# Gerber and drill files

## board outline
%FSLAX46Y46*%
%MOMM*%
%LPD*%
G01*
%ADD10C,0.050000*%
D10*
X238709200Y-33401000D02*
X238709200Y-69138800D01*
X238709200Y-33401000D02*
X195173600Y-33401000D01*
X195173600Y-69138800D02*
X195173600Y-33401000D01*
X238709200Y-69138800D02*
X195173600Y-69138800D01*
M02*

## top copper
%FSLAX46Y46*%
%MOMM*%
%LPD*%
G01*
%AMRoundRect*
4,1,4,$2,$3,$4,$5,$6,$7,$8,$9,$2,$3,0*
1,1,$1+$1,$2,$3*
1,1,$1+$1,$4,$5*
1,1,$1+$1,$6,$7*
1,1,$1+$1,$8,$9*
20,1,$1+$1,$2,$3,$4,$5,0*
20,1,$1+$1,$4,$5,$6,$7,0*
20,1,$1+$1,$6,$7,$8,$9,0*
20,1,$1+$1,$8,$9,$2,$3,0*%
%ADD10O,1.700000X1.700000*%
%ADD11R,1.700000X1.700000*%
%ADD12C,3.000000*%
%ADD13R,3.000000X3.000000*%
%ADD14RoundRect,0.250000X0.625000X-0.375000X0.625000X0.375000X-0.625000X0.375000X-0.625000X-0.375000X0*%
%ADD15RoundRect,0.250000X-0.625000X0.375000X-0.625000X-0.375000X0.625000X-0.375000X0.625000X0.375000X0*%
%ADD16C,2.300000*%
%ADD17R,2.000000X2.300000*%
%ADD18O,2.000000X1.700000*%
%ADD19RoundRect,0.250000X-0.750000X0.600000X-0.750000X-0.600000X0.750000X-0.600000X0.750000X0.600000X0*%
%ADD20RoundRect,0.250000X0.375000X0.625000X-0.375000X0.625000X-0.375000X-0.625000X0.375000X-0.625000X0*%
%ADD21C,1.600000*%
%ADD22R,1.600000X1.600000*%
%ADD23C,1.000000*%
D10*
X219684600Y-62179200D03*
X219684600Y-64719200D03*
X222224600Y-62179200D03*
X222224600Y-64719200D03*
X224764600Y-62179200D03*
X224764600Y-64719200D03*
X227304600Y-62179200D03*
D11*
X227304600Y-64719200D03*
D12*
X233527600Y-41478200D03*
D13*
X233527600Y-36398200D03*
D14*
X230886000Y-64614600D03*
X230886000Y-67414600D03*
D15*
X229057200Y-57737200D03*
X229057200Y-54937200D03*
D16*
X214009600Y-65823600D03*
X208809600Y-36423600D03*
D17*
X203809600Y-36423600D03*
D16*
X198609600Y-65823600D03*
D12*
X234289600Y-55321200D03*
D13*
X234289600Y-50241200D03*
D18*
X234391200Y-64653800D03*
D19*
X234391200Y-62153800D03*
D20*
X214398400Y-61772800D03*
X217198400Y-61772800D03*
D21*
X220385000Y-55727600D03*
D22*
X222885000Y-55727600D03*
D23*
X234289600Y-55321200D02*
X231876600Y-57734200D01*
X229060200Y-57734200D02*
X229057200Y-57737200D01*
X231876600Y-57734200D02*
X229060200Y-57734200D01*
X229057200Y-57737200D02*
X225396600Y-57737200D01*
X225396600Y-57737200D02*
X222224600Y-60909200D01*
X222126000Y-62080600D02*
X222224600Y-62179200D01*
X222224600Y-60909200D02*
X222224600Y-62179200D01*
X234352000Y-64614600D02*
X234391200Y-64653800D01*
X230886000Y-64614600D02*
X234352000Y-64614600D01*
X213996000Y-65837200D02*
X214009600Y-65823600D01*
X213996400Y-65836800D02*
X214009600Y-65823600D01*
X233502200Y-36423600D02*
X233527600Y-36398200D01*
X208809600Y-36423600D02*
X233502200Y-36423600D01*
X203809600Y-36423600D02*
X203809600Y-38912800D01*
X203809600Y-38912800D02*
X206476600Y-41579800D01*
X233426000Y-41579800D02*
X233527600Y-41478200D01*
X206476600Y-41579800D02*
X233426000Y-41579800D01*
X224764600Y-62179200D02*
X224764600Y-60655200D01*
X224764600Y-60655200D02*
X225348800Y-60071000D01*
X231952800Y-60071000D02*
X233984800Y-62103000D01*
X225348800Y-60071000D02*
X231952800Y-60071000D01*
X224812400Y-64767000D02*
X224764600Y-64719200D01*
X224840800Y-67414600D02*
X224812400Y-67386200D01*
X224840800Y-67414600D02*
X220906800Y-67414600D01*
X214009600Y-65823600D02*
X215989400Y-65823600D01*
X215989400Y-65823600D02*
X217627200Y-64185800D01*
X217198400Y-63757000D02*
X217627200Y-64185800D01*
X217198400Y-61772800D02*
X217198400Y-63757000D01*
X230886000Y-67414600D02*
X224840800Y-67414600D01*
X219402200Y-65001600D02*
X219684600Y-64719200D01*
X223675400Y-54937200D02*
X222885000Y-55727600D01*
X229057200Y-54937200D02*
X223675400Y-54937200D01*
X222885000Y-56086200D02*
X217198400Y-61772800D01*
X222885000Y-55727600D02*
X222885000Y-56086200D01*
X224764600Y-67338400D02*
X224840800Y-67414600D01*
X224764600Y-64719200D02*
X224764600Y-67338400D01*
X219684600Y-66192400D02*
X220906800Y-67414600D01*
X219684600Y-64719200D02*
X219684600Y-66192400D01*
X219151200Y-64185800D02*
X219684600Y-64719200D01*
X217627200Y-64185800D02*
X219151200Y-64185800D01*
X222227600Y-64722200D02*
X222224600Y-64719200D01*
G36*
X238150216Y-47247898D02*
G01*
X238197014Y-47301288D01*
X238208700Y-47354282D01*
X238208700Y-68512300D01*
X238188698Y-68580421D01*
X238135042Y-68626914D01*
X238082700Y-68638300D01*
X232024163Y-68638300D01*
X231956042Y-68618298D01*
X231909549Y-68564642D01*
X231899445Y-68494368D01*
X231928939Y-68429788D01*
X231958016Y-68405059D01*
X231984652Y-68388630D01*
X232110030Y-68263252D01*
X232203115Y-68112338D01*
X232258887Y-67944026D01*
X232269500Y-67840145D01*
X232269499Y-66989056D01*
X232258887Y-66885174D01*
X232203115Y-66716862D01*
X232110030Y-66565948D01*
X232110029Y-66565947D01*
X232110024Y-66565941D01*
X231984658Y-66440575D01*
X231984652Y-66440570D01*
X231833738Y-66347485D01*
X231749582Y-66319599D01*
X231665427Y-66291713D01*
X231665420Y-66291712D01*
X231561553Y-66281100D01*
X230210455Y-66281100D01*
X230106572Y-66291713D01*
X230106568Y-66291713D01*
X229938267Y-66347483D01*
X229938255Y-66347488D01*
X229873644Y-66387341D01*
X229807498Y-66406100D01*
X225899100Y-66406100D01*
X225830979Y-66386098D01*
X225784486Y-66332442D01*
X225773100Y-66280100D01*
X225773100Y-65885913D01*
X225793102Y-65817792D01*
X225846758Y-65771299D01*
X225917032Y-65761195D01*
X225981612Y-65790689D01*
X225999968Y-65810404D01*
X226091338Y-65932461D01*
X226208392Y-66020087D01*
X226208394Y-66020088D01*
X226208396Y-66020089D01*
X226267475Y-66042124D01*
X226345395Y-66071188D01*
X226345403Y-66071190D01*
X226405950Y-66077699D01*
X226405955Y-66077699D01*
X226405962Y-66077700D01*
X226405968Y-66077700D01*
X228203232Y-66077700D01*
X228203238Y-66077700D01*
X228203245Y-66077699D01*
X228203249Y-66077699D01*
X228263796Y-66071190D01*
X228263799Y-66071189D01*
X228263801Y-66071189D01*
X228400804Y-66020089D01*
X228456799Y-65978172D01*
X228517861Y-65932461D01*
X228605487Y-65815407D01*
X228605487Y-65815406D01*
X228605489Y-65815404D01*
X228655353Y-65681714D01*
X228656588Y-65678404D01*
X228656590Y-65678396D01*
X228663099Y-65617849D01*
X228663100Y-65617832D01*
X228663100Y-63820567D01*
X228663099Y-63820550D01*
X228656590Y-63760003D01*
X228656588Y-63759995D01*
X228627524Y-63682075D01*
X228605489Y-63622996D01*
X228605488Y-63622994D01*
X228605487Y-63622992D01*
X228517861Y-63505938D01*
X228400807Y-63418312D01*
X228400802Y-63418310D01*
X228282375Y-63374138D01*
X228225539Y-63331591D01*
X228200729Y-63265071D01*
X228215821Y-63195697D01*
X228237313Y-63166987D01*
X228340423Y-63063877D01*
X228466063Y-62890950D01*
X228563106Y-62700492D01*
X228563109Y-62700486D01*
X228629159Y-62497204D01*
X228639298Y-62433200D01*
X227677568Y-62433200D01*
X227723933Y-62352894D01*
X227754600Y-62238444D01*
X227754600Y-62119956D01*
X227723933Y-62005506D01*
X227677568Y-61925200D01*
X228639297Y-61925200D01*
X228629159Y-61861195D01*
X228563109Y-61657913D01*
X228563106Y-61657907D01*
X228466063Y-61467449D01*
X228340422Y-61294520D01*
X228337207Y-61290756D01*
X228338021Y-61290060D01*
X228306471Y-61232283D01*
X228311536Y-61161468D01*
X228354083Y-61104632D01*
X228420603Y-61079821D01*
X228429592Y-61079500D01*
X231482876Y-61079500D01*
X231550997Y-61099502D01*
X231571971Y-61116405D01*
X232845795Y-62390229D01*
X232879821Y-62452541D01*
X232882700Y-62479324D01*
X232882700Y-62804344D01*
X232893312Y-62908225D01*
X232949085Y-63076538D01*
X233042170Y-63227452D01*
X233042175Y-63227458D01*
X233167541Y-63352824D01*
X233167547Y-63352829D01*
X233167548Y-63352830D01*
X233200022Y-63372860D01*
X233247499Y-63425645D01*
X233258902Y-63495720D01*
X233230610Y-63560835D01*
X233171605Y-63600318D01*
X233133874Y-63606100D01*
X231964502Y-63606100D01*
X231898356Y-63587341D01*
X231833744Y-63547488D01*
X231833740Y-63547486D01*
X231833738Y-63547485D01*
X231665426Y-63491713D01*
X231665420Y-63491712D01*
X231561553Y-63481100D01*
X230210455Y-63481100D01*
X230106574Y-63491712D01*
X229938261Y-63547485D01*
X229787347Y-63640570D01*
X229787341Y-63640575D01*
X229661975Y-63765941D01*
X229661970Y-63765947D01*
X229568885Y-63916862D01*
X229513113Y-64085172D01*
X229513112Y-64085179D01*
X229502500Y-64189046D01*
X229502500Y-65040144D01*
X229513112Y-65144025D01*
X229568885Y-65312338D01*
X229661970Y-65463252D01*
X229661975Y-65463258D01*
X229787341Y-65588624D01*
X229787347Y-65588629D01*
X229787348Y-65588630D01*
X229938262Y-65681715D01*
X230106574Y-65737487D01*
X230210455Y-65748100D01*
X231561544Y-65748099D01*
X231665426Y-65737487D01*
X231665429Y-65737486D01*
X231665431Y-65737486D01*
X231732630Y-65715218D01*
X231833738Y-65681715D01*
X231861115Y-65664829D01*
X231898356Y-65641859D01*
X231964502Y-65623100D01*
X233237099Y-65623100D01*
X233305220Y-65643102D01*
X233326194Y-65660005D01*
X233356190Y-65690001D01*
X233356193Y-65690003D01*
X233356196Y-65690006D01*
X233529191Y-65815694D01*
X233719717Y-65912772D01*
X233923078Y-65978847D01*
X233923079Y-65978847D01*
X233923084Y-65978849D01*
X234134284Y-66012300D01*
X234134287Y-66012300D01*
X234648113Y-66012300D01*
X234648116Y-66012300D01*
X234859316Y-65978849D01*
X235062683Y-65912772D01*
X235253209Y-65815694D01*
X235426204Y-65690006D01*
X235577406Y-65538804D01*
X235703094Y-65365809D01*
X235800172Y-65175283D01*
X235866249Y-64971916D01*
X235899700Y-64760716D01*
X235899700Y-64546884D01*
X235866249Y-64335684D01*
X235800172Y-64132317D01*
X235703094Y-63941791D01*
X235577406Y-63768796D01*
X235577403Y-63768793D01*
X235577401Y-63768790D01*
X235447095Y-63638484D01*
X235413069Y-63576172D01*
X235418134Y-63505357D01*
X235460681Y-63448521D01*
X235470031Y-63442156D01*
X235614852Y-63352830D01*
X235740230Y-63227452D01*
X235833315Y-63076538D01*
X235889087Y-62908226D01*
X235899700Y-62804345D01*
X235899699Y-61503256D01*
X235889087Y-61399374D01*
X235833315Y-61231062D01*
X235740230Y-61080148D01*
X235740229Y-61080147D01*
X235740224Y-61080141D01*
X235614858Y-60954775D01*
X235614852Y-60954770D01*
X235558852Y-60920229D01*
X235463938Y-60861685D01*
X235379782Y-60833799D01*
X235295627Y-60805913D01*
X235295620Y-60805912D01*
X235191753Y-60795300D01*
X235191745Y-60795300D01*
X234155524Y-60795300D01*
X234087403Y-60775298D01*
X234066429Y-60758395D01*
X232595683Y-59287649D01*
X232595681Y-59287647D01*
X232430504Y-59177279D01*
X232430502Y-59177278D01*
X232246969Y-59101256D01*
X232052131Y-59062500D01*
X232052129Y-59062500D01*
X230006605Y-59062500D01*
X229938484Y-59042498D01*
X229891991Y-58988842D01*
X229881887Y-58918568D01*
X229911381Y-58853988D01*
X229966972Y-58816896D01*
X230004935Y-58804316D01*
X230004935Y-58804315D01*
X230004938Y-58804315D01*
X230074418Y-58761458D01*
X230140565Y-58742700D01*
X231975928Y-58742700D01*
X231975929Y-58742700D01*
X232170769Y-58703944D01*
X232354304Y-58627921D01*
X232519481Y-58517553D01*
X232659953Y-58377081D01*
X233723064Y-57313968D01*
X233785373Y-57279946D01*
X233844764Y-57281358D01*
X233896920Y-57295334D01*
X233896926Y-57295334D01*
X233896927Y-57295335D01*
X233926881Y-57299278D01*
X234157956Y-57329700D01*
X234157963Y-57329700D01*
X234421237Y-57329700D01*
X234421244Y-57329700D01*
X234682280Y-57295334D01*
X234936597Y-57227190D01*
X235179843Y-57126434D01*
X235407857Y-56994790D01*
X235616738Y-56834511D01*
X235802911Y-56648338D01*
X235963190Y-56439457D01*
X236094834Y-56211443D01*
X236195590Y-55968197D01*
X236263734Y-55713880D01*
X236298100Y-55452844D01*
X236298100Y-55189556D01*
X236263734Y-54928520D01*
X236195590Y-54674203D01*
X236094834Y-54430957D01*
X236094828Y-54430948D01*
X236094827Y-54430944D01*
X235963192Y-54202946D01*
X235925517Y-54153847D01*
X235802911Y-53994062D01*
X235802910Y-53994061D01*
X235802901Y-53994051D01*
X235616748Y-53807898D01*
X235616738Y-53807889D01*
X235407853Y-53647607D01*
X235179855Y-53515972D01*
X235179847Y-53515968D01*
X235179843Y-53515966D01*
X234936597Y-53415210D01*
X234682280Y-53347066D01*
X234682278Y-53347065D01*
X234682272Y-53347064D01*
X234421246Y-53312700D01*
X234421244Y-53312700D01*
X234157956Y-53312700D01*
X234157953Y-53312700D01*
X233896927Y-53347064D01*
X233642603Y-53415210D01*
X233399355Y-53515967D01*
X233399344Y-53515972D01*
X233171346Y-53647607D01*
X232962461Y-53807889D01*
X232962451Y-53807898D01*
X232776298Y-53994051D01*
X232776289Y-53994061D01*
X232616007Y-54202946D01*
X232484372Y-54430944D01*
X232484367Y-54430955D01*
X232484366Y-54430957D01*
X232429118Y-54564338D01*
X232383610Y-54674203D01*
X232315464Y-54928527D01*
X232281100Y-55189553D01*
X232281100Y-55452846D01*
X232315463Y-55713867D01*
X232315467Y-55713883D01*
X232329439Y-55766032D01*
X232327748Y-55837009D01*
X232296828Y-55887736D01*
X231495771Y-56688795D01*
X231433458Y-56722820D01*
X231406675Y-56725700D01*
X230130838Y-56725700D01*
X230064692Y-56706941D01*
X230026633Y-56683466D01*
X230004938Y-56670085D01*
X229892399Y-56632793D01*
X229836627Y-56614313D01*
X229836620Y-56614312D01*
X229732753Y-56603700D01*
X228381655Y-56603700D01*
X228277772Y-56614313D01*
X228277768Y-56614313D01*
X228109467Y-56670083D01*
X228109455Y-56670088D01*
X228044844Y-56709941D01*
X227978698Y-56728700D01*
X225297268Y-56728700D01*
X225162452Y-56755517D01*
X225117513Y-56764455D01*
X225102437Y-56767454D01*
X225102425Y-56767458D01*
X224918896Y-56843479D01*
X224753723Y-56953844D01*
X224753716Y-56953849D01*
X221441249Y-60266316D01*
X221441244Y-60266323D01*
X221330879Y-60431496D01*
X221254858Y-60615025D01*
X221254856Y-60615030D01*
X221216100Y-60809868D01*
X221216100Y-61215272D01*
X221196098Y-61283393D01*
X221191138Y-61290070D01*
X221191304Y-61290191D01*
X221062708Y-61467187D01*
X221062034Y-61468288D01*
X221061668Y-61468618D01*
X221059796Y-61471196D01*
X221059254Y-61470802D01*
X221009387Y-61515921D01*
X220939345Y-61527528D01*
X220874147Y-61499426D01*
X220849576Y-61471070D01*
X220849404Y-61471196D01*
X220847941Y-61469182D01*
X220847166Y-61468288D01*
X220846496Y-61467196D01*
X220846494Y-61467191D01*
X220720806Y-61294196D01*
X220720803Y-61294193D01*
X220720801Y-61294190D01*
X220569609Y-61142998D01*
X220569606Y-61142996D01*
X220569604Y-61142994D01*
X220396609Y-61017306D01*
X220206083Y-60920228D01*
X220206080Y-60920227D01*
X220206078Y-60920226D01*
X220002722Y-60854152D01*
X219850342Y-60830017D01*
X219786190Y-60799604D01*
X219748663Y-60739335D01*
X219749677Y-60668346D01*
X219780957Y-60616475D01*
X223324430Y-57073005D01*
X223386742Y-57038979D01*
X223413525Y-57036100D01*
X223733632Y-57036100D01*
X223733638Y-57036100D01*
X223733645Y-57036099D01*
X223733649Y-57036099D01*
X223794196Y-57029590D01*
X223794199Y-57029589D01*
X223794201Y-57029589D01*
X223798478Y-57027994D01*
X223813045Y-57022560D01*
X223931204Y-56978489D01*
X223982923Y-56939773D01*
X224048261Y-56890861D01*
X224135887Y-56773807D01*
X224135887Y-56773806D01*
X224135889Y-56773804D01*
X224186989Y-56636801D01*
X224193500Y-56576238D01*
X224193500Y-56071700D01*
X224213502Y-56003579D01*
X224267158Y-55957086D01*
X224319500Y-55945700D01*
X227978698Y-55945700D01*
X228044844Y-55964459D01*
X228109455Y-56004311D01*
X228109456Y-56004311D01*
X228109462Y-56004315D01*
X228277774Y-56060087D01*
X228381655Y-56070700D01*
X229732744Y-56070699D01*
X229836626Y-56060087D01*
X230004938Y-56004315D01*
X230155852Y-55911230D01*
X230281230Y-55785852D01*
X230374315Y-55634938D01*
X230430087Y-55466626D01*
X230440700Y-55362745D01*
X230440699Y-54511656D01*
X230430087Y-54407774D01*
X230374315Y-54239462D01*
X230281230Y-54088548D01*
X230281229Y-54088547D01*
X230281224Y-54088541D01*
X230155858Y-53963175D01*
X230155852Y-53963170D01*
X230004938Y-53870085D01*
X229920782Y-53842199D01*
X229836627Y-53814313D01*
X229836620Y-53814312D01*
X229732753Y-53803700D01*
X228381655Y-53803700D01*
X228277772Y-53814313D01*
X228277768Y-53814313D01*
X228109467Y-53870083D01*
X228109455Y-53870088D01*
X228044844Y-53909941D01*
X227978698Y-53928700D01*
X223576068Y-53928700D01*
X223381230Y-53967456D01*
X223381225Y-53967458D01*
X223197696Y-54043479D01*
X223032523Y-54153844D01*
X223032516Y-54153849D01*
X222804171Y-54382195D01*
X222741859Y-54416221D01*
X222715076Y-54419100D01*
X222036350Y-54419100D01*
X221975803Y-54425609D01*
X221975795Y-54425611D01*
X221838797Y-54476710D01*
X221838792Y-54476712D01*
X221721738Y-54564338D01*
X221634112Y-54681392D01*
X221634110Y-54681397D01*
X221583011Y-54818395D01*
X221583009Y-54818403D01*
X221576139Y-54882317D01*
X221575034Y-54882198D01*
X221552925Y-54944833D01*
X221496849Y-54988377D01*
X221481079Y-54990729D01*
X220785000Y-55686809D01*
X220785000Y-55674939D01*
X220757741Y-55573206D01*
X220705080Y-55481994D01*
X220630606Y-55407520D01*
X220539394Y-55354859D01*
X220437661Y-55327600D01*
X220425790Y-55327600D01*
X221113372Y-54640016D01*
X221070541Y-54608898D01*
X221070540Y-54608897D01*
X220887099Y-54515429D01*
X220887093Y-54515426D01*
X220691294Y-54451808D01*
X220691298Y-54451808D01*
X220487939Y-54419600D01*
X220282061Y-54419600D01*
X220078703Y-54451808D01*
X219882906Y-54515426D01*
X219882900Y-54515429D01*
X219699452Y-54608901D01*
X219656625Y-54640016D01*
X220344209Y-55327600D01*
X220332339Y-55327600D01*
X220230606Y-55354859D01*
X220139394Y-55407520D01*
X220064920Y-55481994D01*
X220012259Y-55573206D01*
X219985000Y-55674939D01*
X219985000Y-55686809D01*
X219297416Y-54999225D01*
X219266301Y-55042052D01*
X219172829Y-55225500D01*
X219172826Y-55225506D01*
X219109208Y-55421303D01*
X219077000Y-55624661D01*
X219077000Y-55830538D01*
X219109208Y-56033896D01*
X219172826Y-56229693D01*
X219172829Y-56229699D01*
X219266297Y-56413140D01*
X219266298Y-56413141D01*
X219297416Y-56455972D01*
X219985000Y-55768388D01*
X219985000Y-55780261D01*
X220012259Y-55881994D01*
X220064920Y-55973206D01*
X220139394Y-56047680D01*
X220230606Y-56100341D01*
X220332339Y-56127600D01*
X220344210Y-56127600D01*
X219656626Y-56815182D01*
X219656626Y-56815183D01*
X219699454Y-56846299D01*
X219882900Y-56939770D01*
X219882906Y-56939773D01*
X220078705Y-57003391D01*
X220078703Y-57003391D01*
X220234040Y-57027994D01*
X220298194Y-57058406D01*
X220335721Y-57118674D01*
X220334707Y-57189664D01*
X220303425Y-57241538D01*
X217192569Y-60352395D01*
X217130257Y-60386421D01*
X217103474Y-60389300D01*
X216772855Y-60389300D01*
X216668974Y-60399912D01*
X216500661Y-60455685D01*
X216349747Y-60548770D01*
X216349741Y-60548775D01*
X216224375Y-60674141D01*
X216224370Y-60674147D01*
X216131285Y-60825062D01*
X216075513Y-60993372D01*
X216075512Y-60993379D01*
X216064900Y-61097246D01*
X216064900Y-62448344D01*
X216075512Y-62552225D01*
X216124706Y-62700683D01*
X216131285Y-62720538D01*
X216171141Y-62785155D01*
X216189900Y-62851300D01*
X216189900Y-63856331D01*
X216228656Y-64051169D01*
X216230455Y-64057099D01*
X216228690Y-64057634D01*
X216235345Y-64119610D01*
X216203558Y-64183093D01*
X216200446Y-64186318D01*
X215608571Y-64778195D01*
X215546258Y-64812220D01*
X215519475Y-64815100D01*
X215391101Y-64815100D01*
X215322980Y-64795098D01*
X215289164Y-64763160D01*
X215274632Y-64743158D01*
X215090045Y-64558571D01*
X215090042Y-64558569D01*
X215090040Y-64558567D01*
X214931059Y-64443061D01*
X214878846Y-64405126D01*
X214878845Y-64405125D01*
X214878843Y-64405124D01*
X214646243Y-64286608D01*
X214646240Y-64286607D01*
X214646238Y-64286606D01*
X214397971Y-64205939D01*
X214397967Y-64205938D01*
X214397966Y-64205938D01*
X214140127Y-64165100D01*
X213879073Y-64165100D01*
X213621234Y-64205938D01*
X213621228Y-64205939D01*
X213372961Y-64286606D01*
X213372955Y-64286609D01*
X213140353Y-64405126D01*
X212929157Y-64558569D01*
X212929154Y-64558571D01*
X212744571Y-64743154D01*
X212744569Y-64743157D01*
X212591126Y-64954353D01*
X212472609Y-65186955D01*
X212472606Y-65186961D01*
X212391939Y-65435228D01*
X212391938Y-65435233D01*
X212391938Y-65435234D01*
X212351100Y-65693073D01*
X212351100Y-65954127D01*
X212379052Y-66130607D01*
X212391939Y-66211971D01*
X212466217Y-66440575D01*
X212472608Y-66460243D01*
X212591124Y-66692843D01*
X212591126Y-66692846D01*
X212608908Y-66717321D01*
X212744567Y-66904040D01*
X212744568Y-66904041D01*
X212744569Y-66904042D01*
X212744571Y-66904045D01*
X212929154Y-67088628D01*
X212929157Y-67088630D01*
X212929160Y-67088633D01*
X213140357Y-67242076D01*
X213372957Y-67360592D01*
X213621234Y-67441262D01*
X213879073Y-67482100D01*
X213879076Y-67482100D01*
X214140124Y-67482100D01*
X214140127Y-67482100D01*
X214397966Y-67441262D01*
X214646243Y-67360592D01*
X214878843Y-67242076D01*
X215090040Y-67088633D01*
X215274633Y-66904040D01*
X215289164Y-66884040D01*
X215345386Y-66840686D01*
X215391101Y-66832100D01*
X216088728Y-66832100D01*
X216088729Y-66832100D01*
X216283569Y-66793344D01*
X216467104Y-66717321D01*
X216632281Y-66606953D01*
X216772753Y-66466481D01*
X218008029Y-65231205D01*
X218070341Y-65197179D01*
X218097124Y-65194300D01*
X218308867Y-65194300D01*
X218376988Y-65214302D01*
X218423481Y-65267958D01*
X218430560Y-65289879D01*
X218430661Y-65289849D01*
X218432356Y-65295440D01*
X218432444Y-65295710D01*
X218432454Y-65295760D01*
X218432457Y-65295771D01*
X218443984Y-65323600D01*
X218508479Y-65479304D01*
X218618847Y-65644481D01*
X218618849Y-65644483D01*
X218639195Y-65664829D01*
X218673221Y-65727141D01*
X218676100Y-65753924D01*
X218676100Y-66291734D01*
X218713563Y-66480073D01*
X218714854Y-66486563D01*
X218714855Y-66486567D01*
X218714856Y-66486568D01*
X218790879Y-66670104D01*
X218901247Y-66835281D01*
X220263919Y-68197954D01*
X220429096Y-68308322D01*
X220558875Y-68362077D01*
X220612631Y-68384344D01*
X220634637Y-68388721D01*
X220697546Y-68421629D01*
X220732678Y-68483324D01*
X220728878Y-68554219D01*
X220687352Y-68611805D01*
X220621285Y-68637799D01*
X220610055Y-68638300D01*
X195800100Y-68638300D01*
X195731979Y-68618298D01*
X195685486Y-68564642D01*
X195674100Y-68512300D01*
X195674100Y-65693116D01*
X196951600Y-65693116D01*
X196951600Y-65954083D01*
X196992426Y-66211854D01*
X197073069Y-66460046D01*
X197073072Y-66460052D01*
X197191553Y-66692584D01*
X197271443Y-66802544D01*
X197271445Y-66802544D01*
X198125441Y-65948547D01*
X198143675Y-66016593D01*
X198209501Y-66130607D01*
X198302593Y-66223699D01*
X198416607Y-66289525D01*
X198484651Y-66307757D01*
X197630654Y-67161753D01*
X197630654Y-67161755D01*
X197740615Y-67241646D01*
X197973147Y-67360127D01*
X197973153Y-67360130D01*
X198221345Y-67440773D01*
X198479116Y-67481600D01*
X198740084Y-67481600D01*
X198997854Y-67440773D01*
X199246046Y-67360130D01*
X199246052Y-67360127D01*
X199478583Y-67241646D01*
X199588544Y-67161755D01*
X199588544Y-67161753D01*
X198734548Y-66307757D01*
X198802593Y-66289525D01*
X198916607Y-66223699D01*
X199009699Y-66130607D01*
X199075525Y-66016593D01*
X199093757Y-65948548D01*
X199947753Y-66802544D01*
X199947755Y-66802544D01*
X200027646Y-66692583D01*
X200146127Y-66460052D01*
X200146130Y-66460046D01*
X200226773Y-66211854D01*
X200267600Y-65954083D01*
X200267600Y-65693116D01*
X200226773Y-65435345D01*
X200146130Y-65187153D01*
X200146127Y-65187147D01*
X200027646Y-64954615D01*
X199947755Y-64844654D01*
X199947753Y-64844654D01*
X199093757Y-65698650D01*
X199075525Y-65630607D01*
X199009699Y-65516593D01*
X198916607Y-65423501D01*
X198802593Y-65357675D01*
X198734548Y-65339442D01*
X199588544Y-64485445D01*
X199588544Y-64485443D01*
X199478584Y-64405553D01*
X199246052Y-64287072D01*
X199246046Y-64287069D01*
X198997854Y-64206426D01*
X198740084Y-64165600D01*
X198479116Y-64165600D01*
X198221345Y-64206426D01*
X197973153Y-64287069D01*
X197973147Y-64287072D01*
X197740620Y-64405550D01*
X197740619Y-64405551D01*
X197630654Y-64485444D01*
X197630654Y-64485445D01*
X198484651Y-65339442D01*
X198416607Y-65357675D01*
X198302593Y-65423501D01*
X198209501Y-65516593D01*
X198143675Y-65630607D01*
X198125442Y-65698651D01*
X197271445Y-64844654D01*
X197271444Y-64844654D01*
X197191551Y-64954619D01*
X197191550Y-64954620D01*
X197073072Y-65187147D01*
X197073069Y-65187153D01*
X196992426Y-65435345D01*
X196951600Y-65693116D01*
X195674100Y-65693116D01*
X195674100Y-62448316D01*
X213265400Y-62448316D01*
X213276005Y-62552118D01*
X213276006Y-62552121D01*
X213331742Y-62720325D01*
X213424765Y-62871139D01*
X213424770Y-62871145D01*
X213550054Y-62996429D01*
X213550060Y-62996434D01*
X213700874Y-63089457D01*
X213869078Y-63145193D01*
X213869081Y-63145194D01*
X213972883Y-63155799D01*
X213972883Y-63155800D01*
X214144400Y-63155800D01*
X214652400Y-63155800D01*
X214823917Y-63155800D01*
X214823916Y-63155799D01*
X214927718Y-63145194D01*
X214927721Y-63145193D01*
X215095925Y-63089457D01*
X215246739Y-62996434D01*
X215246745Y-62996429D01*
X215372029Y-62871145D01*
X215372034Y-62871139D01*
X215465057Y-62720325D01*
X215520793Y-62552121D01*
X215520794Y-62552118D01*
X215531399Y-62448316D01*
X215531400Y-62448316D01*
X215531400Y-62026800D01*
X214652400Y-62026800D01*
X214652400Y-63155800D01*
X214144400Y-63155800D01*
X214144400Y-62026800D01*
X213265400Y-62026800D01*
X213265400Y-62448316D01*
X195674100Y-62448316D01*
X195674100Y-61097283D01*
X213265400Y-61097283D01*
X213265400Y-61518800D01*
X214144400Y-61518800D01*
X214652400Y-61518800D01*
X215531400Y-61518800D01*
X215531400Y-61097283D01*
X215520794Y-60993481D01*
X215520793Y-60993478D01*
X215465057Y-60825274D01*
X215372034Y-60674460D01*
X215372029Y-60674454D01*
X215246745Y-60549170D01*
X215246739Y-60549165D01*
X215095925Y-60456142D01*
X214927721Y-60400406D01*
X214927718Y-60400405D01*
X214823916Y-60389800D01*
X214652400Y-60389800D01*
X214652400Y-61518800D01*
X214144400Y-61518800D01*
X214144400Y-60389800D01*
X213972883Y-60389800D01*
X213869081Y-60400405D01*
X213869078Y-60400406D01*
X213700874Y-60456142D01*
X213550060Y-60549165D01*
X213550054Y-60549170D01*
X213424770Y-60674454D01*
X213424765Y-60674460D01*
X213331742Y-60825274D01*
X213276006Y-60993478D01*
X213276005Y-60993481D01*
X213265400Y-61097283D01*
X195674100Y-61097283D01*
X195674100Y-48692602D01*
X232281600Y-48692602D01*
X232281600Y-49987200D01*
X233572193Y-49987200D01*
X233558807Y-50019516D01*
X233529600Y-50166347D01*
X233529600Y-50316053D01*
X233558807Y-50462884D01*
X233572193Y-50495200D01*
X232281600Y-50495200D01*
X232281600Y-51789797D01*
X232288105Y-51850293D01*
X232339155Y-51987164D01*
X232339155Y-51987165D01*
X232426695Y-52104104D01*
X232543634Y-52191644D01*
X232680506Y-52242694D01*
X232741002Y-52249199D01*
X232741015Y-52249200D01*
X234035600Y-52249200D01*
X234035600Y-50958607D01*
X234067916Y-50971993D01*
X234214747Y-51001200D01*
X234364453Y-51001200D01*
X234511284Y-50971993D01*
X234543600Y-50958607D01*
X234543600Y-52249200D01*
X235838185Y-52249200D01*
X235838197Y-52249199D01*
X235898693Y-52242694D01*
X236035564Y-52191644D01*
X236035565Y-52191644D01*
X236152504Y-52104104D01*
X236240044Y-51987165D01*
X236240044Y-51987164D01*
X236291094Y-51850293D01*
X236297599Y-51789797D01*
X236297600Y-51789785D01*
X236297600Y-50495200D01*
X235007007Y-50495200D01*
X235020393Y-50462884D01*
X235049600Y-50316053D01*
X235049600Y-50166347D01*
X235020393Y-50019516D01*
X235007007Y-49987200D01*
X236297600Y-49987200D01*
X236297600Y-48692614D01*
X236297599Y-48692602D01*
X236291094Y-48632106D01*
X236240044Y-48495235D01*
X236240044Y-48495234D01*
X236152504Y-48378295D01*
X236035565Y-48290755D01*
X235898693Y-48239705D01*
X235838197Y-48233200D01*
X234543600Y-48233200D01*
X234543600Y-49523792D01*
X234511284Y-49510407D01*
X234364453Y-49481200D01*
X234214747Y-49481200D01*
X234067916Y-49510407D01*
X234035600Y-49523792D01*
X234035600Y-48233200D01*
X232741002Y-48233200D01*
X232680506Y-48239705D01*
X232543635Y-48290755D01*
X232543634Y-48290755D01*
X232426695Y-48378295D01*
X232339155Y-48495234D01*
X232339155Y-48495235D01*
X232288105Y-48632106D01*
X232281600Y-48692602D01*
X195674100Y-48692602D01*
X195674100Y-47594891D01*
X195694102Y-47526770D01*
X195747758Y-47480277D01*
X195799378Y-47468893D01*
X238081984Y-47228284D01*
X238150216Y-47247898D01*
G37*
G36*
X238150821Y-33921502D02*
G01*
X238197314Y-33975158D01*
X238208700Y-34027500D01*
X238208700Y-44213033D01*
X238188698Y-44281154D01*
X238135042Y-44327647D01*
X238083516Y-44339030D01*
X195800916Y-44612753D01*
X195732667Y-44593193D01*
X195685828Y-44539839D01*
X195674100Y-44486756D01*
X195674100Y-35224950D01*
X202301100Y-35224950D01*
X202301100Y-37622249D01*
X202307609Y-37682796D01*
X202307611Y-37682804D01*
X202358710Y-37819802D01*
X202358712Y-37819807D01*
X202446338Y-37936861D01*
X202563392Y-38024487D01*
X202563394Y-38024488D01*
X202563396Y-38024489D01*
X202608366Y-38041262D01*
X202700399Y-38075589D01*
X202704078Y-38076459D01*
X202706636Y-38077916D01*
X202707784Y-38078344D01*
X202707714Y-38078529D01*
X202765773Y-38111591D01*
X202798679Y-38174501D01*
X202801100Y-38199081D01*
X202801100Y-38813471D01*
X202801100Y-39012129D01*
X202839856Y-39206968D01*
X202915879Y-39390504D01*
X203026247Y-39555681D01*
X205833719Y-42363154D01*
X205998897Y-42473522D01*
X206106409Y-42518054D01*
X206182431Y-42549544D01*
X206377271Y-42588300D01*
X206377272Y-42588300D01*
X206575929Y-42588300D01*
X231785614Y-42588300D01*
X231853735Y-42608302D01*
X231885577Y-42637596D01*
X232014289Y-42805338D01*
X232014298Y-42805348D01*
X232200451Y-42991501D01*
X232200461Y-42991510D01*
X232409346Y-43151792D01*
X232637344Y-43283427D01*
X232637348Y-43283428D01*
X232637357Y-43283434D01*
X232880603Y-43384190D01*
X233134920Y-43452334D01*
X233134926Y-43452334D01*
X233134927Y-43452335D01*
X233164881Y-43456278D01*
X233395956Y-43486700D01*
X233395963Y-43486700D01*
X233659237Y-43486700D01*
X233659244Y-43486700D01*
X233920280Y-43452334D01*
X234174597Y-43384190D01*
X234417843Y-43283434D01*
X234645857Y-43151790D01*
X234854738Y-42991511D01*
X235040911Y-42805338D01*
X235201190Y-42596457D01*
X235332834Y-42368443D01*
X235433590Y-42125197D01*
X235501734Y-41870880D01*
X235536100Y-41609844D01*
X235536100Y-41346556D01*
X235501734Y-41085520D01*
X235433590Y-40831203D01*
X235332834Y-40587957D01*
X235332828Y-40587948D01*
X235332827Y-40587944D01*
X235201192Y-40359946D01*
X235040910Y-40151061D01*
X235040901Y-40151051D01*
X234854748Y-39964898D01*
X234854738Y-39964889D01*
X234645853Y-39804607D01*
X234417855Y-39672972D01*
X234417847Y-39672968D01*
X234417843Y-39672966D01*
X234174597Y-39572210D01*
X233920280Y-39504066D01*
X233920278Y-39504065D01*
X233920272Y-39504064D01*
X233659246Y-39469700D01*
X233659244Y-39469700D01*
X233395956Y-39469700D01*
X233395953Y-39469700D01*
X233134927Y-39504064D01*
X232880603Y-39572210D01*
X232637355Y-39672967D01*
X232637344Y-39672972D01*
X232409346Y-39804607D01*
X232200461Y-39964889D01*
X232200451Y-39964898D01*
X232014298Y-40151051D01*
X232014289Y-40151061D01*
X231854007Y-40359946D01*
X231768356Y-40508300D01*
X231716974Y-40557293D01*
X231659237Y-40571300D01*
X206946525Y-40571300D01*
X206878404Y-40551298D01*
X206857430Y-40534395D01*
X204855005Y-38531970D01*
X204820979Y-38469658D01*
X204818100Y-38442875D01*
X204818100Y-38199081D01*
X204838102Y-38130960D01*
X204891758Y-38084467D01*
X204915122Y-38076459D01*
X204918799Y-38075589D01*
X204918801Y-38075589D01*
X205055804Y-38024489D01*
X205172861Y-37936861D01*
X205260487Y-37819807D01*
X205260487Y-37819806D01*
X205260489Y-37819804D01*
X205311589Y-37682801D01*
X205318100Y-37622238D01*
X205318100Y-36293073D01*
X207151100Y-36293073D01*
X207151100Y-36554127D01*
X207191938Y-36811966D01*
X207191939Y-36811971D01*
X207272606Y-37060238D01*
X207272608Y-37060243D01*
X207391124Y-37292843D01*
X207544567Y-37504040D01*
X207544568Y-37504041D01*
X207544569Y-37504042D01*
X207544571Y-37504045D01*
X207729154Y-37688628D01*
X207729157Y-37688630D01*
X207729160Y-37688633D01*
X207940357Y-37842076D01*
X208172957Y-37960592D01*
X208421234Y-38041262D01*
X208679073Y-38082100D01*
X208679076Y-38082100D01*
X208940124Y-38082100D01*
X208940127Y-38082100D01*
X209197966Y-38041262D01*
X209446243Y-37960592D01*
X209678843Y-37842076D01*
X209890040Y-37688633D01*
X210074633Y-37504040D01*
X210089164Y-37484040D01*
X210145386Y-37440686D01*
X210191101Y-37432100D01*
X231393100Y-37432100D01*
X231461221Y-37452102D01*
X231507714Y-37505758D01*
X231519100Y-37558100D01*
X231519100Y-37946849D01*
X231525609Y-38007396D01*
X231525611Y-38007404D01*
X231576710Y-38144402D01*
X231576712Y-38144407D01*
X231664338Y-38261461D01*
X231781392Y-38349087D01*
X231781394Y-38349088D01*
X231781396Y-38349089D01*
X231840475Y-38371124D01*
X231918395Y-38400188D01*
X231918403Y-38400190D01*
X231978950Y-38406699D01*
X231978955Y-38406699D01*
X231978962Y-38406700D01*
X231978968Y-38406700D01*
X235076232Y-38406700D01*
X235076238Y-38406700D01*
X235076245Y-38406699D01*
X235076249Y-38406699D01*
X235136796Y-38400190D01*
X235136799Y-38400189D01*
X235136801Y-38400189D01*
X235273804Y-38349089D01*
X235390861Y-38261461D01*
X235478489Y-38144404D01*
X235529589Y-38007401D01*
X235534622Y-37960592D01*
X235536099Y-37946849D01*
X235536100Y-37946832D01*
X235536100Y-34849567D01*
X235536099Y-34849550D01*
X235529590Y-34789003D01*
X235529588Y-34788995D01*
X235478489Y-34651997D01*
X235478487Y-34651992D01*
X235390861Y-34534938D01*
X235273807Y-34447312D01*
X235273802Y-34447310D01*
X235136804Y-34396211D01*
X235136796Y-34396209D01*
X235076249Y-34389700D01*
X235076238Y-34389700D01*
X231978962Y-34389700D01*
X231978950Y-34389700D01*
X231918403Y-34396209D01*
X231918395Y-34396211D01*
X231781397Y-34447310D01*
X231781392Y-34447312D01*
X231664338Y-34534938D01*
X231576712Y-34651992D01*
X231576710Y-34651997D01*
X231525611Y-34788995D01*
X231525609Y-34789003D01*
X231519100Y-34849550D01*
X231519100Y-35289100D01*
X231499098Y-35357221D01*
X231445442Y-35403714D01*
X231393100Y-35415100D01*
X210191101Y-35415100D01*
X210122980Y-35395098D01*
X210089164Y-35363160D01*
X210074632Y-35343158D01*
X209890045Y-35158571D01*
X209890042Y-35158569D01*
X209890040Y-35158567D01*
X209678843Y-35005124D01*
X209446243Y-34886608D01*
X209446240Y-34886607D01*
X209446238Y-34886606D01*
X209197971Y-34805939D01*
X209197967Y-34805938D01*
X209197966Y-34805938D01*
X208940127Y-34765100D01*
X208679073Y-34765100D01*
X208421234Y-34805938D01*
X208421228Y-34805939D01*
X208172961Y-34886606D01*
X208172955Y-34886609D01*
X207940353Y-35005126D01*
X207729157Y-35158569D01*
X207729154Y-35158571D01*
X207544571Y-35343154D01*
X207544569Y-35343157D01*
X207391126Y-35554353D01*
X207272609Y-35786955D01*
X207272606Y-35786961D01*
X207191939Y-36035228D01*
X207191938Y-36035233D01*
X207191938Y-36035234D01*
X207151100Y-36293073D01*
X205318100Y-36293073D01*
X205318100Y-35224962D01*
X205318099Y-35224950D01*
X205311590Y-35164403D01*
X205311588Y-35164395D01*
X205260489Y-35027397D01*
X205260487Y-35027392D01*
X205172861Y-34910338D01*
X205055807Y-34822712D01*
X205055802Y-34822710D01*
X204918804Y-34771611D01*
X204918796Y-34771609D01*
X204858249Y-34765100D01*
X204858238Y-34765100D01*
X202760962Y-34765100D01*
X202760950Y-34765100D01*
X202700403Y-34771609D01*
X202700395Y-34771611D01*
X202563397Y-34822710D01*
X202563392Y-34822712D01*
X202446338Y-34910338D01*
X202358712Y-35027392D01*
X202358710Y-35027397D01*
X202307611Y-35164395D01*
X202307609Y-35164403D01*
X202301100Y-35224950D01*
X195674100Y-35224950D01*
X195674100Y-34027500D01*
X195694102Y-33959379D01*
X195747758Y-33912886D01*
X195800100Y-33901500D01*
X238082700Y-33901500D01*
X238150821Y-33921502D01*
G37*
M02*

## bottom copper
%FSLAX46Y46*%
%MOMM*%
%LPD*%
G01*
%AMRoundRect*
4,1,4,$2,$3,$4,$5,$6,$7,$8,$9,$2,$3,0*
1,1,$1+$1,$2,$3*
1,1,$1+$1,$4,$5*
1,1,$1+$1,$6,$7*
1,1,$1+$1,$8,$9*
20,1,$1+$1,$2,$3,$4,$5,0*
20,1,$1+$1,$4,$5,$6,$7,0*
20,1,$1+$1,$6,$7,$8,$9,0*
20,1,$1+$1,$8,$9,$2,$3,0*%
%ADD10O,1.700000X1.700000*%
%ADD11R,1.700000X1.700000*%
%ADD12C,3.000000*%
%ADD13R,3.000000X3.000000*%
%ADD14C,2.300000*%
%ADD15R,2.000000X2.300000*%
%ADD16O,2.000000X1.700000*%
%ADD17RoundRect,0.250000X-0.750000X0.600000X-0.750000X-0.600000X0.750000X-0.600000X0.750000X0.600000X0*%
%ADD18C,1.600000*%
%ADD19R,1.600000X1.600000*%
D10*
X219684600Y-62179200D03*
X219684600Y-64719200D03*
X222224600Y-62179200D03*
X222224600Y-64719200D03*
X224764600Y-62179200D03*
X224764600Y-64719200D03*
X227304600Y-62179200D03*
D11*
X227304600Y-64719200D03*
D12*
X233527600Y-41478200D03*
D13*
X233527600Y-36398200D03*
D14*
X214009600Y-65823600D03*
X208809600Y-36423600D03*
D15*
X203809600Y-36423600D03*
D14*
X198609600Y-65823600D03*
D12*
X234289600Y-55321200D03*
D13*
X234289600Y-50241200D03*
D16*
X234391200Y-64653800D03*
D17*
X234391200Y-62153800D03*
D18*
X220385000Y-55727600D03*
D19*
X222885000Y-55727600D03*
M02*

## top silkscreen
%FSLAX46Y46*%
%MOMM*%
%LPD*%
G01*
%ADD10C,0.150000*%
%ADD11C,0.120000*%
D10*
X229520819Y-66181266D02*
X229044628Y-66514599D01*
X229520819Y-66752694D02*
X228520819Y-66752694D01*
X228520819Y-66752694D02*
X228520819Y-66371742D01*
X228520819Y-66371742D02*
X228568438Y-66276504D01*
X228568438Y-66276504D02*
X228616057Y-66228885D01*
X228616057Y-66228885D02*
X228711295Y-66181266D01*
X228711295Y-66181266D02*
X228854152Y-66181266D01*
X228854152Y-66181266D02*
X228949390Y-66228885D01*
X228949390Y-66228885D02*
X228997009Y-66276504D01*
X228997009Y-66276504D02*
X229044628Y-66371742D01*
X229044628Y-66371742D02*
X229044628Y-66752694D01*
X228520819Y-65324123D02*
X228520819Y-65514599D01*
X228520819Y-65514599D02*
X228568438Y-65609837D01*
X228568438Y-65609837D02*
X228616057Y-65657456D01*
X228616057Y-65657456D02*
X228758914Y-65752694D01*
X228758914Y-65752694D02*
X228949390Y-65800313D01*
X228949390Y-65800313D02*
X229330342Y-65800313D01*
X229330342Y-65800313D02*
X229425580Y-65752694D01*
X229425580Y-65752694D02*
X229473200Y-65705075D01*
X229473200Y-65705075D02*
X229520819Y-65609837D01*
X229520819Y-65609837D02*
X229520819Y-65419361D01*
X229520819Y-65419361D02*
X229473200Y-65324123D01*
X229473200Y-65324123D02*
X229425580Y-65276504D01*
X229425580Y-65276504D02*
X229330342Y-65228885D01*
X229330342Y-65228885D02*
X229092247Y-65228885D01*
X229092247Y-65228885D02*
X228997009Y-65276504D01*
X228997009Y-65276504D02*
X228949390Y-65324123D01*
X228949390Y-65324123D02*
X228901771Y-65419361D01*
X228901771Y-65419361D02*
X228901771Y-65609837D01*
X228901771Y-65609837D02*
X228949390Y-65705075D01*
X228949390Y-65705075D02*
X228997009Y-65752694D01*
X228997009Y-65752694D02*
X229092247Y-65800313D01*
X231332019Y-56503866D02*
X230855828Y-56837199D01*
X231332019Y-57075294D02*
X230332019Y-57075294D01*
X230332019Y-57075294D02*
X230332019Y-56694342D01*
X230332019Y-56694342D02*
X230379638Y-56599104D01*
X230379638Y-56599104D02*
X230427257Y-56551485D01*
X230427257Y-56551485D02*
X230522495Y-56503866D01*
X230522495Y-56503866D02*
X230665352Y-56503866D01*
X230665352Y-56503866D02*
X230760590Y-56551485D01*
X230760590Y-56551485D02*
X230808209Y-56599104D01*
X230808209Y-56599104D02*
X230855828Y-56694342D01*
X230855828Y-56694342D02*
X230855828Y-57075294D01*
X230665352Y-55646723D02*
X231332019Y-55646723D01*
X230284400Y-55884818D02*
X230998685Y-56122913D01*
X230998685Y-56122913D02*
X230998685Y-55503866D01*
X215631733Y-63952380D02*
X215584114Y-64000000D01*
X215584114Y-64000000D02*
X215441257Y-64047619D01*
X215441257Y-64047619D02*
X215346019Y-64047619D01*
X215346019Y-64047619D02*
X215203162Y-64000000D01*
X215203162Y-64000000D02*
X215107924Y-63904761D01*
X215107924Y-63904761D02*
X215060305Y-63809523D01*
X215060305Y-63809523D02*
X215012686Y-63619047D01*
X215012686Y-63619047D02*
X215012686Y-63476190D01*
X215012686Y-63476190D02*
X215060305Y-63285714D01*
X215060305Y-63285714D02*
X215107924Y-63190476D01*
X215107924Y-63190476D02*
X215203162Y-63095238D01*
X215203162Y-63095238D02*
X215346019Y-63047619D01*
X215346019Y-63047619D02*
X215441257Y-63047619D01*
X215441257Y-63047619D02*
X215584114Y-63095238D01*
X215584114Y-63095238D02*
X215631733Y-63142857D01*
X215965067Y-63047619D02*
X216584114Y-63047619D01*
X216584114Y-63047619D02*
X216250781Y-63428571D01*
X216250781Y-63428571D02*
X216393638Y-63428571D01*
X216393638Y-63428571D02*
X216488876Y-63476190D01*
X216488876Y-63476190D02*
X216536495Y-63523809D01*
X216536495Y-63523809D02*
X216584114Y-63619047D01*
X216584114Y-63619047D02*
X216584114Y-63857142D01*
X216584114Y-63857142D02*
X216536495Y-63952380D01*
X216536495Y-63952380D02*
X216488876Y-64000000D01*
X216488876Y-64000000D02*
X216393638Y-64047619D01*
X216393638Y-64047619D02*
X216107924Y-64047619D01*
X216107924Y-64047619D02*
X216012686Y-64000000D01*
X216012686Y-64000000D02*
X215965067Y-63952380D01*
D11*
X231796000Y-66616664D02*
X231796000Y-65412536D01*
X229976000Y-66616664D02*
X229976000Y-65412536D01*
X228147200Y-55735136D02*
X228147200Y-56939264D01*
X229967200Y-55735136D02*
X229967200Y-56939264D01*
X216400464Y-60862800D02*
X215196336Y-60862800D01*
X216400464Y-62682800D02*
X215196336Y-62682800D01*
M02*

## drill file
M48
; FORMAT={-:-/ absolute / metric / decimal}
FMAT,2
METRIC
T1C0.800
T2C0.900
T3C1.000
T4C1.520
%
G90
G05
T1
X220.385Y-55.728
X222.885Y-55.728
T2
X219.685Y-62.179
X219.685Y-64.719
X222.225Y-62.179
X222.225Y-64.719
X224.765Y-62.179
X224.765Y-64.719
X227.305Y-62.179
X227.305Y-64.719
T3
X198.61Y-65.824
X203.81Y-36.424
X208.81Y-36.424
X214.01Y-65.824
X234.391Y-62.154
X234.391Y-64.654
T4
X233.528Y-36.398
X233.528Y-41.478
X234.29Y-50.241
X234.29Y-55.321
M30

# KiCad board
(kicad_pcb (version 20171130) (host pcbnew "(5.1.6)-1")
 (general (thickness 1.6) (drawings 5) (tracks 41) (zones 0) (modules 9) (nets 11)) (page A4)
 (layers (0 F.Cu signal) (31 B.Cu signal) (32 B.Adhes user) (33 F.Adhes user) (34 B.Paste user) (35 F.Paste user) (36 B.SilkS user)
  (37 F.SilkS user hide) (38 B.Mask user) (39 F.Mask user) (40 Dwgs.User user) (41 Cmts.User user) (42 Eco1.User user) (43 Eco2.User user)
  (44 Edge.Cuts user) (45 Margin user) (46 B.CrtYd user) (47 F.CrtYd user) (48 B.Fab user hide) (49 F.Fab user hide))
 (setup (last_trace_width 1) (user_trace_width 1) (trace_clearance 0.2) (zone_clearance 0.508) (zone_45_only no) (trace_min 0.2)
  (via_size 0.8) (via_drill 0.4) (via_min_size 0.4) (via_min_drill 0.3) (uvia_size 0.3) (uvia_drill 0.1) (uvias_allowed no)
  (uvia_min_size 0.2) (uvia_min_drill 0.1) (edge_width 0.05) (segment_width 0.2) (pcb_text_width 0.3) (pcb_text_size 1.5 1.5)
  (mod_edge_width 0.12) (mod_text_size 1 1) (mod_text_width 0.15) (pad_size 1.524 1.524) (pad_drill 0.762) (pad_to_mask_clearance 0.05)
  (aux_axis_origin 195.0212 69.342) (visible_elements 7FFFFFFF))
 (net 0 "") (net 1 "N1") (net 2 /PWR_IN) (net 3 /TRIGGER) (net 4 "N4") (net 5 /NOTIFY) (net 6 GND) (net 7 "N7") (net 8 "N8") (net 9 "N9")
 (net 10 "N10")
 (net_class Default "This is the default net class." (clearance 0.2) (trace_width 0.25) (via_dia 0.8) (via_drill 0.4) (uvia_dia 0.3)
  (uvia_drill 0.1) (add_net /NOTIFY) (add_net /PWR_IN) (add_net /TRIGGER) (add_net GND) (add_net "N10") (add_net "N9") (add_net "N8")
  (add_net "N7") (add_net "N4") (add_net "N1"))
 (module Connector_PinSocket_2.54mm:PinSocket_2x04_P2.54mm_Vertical (layer B.Cu) (at 227.3046 62.1792 90)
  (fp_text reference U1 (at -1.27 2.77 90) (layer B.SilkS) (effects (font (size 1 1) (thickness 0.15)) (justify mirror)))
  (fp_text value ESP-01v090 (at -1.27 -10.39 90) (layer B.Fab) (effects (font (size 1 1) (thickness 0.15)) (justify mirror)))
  (pad 8 thru_hole oval (at 0 -7.62 90) (size 1.7 1.7) (drill 0.9) (layers *.Cu *.Mask) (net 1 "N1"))
  (pad 7 thru_hole oval (at -2.54 -7.62 90) (size 1.7 1.7) (drill 0.9) (layers *.Cu *.Mask) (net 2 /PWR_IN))
  (pad 6 thru_hole oval (at 0 -5.08 90) (size 1.7 1.7) (drill 0.9) (layers *.Cu *.Mask) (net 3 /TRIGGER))
  (pad 5 thru_hole oval (at -2.54 -5.08 90) (size 1.7 1.7) (drill 0.9) (layers *.Cu *.Mask) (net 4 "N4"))
  (pad 4 thru_hole oval (at 0 -2.54 90) (size 1.7 1.7) (drill 0.9) (layers *.Cu *.Mask) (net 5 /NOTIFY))
  (pad 3 thru_hole oval (at -2.54 -2.54 90) (size 1.7 1.7) (drill 0.9) (layers *.Cu *.Mask) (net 2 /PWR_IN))
  (pad 2 thru_hole oval (at 0 0 90) (size 1.7 1.7) (drill 0.9) (layers *.Cu *.Mask) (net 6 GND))
  (pad 1 thru_hole rect (at -2.54 0 90) (size 1.7 1.7) (drill 0.9) (layers *.Cu *.Mask) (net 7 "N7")))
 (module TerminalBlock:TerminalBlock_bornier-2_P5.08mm (layer B.Cu) (at 233.5276 36.3982 270)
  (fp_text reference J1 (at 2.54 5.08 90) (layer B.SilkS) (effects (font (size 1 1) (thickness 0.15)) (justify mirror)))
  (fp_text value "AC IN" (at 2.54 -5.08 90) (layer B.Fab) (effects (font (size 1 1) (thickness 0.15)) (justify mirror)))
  (pad 2 thru_hole circle (at 5.08 0 270) (size 3 3) (drill 1.52) (layers *.Cu *.Mask) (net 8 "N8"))
  (pad 1 thru_hole rect (at 0 0 270) (size 3 3) (drill 1.52) (layers *.Cu *.Mask) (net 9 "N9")))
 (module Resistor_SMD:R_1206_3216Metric (layer F.Cu) (at 230.886 66.0146 90)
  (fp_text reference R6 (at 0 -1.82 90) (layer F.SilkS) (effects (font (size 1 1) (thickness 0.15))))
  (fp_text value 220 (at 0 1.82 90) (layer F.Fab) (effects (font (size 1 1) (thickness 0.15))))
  (fp_line (start -0.602064 0.91) (end 0.602064 0.91) (layer F.SilkS) (width 0.12))
  (fp_line (start -0.602064 -0.91) (end 0.602064 -0.91) (layer F.SilkS) (width 0.12))
  (pad 2 smd roundrect (at 1.4 0 90) (size 1.25 1.75) (layers F.Cu F.Paste F.Mask) (roundrect_rratio 0.2) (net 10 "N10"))
  (pad 1 smd roundrect (at -1.4 0 90) (size 1.25 1.75) (layers F.Cu F.Paste F.Mask) (roundrect_rratio 0.2) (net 2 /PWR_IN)))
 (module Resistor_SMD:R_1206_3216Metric (layer F.Cu) (at 229.0572 56.3372 270)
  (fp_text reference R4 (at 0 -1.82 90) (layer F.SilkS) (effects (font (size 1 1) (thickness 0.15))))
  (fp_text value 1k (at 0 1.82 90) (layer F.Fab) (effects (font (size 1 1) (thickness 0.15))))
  (fp_line (start -0.602064 0.91) (end 0.602064 0.91) (layer F.SilkS) (width 0.12))
  (fp_line (start -0.602064 -0.91) (end 0.602064 -0.91) (layer F.SilkS) (width 0.12))
  (pad 2 smd roundrect (at 1.4 0 270) (size 1.25 1.75) (layers F.Cu F.Paste F.Mask) (roundrect_rratio 0.2) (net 3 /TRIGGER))
  (pad 1 smd roundrect (at -1.4 0 270) (size 1.25 1.75) (layers F.Cu F.Paste F.Mask) (roundrect_rratio 0.2) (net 2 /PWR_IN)))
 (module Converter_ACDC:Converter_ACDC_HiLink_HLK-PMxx (layer B.Cu) (at 203.8096 36.4236 270)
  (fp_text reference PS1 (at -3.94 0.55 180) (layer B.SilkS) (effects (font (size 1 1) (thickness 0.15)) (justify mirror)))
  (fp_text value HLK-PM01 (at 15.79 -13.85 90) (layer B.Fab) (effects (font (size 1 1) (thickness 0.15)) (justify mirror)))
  (pad 4 thru_hole circle (at 29.4 -10.2 270) (size 2.3 2.3) (drill 1) (layers *.Cu *.Mask) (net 2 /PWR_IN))
  (pad 2 thru_hole circle (at 0 -5 270) (size 2.3 2.3) (drill 1) (layers *.Cu *.Mask) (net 9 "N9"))
  (pad 1 thru_hole rect (at 0 0 270) (size 2.3 2) (drill 1) (layers *.Cu *.Mask) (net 8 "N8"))
  (pad 3 thru_hole circle (at 29.4 5.2 270) (size 2.3 2.3) (drill 1) (layers *.Cu *.Mask) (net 6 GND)))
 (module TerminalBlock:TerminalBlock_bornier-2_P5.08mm (layer B.Cu) (at 234.2896 50.2412 270)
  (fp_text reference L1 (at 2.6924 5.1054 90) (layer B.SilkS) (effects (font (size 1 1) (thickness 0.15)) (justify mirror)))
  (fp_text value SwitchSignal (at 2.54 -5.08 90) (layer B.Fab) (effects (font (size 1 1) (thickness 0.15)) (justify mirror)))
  (pad 2 thru_hole circle (at 5.08 0 270) (size 3 3) (drill 1.52) (layers *.Cu *.Mask) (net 3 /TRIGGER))
  (pad 1 thru_hole rect (at 0 0 270) (size 3 3) (drill 1.52) (layers *.Cu *.Mask) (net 6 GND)))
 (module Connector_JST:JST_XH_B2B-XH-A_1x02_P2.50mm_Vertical (layer B.Cu) (at 234.3912 62.1538 270)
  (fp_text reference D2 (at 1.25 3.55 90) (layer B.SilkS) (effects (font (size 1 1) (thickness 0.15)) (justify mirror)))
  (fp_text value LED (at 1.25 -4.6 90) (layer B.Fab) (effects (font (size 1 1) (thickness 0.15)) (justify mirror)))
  (pad 2 thru_hole oval (at 2.5 0 270) (size 1.7 2) (drill 1) (layers *.Cu *.Mask) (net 10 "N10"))
  (pad 1 thru_hole roundrect (at 0 0 270) (size 1.7 2) (drill 1) (layers *.Cu *.Mask) (roundrect_rratio 0.147059) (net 5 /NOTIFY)))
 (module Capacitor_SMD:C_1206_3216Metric (layer F.Cu) (at 215.7984 61.7728 180)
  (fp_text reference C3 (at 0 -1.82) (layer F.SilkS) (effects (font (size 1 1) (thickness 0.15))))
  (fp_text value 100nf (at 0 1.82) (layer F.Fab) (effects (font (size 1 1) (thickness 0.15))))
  (fp_line (start -0.602064 0.91) (end 0.602064 0.91) (layer F.SilkS) (width 0.12))
  (fp_line (start -0.602064 -0.91) (end 0.602064 -0.91) (layer F.SilkS) (width 0.12))
  (pad 2 smd roundrect (at 1.4 0 180) (size 1.25 1.75) (layers F.Cu F.Paste F.Mask) (roundrect_rratio 0.2) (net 6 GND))
  (pad 1 smd roundrect (at -1.4 0 180) (size 1.25 1.75) (layers F.Cu F.Paste F.Mask) (roundrect_rratio 0.2) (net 2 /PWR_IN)))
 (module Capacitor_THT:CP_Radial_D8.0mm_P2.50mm (layer B.Cu) (at 222.885 55.7276 180)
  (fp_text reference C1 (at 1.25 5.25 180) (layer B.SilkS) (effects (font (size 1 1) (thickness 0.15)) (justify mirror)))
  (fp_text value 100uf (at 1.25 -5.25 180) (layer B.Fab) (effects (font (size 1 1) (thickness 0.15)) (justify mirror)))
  (pad 2 thru_hole circle (at 2.5 0 180) (size 1.6 1.6) (drill 0.8) (layers *.Cu *.Mask) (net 6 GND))
  (pad 1 thru_hole rect (at 0 0 180) (size 1.6 1.6) (drill 0.8) (layers *.Cu *.Mask) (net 2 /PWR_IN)))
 (gr_line (start 238.7092 33.401) (end 238.7092 69.1388) (layer Edge.Cuts) (width 0.05))
 (gr_line (start 238.7092 33.401) (end 195.1736 33.401) (layer Edge.Cuts) (width 0.05))
 (gr_line (start 195.1736 69.1388) (end 195.1736 33.401) (layer Edge.Cuts) (width 0.05))
 (gr_line (start 238.7092 69.1388) (end 195.1736 69.1388) (layer Edge.Cuts) (width 0.05))
 (segment (start 234.2896 55.3212) (end 231.8766 57.7342) (width 1) (layer F.Cu) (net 3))
 (segment (start 229.0602 57.7342) (end 229.0572 57.7372) (width 1) (layer F.Cu) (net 3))
 (segment (start 231.8766 57.7342) (end 229.0602 57.7342) (width 1) (layer F.Cu) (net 3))
 (segment (start 229.0572 57.7372) (end 225.3966 57.7372) (width 1) (layer F.Cu) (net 3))
 (segment (start 225.3966 57.7372) (end 222.2246 60.9092) (width 1) (layer F.Cu) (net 3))
 (segment (start 222.126 62.0806) (end 222.2246 62.1792) (width 1) (layer F.Cu) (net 3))
 (segment (start 222.2246 60.9092) (end 222.2246 62.1792) (width 1) (layer F.Cu) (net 3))
 (segment (start 234.352 64.6146) (end 234.3912 64.6538) (width 1) (layer F.Cu) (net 10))
 (segment (start 230.886 64.6146) (end 234.352 64.6146) (width 1) (layer F.Cu) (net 10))
 (segment (start 213.996 65.8372) (end 214.0096 65.8236) (width 1) (layer F.Cu) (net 2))
 (segment (start 213.9964 65.8368) (end 214.0096 65.8236) (width 1) (layer F.Cu) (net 2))
 (segment (start 233.5022 36.4236) (end 233.5276 36.3982) (width 1) (layer F.Cu) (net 9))
 (segment (start 208.8096 36.4236) (end 233.5022 36.4236) (width 1) (layer F.Cu) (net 9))
 (segment (start 203.8096 36.4236) (end 203.8096 38.9128) (width 1) (layer F.Cu) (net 8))
 (segment (start 203.8096 38.9128) (end 206.4766 41.5798) (width 1) (layer F.Cu) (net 8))
 (segment (start 233.426 41.5798) (end 233.5276 41.4782) (width 1) (layer F.Cu) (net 8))
 (segment (start 206.4766 41.5798) (end 233.426 41.5798) (width 1) (layer F.Cu) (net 8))
 (segment (start 224.7646 62.1792) (end 224.7646 60.6552) (width 1) (layer F.Cu) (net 5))
 (segment (start 224.7646 60.6552) (end 225.3488 60.071) (width 1) (layer F.Cu) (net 5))
 (segment (start 231.9528 60.071) (end 233.9848 62.103) (width 1) (layer F.Cu) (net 5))
 (segment (start 225.3488 60.071) (end 231.9528 60.071) (width 1) (layer F.Cu) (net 5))
 (segment (start 224.8124 64.767) (end 224.7646 64.7192) (width 1) (layer F.Cu) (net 2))
 (segment (start 224.8408 67.4146) (end 224.8124 67.3862) (width 1) (layer F.Cu) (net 2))
 (segment (start 224.8408 67.4146) (end 220.9068 67.4146) (width 1) (layer F.Cu) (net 2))
 (segment (start 214.0096 65.8236) (end 215.9894 65.8236) (width 1) (layer F.Cu) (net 2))
 (segment (start 215.9894 65.8236) (end 217.6272 64.1858) (width 1) (layer F.Cu) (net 2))
 (segment (start 217.1984 63.757) (end 217.6272 64.1858) (width 1) (layer F.Cu) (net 2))
 (segment (start 217.1984 61.7728) (end 217.1984 63.757) (width 1) (layer F.Cu) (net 2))
 (segment (start 230.886 67.4146) (end 224.8408 67.4146) (width 1) (layer F.Cu) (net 2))
 (segment (start 219.4022 65.0016) (end 219.6846 64.7192) (width 1) (layer F.Cu) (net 2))
 (segment (start 223.6754 54.9372) (end 222.885 55.7276) (width 1) (layer F.Cu) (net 2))
 (segment (start 229.0572 54.9372) (end 223.6754 54.9372) (width 1) (layer F.Cu) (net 2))
 (segment (start 222.885 56.0862) (end 217.1984 61.7728) (width 1) (layer F.Cu) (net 2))
 (segment (start 222.885 55.7276) (end 222.885 56.0862) (width 1) (layer F.Cu) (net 2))
 (segment (start 224.7646 67.3384) (end 224.8408 67.4146) (width 1) (layer F.Cu) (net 2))
 (segment (start 224.7646 64.7192) (end 224.7646 67.3384) (width 1) (layer F.Cu) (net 2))
 (segment (start 219.6846 66.1924) (end 220.9068 67.4146) (width 1) (layer F.Cu) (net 2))
 (segment (start 219.6846 64.7192) (end 219.6846 66.1924) (width 1) (layer F.Cu) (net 2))
 (segment (start 219.1512 64.1858) (end 219.6846 64.7192) (width 1) (layer F.Cu) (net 2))
 (segment (start 217.6272 64.1858) (end 219.1512 64.1858) (width 1) (layer F.Cu) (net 2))
 (segment (start 222.2276 64.7222) (end 222.2246 64.7192) (width 1) (layer F.Cu) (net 4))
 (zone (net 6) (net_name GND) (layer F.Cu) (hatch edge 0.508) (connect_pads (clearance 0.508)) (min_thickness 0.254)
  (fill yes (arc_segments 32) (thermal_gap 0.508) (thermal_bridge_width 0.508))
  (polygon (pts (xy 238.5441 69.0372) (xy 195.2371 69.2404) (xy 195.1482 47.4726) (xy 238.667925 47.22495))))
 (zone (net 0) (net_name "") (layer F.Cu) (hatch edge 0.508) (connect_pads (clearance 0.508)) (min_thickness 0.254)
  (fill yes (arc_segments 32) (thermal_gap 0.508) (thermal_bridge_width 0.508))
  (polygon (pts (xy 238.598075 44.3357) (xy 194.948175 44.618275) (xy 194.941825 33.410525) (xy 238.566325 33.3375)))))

